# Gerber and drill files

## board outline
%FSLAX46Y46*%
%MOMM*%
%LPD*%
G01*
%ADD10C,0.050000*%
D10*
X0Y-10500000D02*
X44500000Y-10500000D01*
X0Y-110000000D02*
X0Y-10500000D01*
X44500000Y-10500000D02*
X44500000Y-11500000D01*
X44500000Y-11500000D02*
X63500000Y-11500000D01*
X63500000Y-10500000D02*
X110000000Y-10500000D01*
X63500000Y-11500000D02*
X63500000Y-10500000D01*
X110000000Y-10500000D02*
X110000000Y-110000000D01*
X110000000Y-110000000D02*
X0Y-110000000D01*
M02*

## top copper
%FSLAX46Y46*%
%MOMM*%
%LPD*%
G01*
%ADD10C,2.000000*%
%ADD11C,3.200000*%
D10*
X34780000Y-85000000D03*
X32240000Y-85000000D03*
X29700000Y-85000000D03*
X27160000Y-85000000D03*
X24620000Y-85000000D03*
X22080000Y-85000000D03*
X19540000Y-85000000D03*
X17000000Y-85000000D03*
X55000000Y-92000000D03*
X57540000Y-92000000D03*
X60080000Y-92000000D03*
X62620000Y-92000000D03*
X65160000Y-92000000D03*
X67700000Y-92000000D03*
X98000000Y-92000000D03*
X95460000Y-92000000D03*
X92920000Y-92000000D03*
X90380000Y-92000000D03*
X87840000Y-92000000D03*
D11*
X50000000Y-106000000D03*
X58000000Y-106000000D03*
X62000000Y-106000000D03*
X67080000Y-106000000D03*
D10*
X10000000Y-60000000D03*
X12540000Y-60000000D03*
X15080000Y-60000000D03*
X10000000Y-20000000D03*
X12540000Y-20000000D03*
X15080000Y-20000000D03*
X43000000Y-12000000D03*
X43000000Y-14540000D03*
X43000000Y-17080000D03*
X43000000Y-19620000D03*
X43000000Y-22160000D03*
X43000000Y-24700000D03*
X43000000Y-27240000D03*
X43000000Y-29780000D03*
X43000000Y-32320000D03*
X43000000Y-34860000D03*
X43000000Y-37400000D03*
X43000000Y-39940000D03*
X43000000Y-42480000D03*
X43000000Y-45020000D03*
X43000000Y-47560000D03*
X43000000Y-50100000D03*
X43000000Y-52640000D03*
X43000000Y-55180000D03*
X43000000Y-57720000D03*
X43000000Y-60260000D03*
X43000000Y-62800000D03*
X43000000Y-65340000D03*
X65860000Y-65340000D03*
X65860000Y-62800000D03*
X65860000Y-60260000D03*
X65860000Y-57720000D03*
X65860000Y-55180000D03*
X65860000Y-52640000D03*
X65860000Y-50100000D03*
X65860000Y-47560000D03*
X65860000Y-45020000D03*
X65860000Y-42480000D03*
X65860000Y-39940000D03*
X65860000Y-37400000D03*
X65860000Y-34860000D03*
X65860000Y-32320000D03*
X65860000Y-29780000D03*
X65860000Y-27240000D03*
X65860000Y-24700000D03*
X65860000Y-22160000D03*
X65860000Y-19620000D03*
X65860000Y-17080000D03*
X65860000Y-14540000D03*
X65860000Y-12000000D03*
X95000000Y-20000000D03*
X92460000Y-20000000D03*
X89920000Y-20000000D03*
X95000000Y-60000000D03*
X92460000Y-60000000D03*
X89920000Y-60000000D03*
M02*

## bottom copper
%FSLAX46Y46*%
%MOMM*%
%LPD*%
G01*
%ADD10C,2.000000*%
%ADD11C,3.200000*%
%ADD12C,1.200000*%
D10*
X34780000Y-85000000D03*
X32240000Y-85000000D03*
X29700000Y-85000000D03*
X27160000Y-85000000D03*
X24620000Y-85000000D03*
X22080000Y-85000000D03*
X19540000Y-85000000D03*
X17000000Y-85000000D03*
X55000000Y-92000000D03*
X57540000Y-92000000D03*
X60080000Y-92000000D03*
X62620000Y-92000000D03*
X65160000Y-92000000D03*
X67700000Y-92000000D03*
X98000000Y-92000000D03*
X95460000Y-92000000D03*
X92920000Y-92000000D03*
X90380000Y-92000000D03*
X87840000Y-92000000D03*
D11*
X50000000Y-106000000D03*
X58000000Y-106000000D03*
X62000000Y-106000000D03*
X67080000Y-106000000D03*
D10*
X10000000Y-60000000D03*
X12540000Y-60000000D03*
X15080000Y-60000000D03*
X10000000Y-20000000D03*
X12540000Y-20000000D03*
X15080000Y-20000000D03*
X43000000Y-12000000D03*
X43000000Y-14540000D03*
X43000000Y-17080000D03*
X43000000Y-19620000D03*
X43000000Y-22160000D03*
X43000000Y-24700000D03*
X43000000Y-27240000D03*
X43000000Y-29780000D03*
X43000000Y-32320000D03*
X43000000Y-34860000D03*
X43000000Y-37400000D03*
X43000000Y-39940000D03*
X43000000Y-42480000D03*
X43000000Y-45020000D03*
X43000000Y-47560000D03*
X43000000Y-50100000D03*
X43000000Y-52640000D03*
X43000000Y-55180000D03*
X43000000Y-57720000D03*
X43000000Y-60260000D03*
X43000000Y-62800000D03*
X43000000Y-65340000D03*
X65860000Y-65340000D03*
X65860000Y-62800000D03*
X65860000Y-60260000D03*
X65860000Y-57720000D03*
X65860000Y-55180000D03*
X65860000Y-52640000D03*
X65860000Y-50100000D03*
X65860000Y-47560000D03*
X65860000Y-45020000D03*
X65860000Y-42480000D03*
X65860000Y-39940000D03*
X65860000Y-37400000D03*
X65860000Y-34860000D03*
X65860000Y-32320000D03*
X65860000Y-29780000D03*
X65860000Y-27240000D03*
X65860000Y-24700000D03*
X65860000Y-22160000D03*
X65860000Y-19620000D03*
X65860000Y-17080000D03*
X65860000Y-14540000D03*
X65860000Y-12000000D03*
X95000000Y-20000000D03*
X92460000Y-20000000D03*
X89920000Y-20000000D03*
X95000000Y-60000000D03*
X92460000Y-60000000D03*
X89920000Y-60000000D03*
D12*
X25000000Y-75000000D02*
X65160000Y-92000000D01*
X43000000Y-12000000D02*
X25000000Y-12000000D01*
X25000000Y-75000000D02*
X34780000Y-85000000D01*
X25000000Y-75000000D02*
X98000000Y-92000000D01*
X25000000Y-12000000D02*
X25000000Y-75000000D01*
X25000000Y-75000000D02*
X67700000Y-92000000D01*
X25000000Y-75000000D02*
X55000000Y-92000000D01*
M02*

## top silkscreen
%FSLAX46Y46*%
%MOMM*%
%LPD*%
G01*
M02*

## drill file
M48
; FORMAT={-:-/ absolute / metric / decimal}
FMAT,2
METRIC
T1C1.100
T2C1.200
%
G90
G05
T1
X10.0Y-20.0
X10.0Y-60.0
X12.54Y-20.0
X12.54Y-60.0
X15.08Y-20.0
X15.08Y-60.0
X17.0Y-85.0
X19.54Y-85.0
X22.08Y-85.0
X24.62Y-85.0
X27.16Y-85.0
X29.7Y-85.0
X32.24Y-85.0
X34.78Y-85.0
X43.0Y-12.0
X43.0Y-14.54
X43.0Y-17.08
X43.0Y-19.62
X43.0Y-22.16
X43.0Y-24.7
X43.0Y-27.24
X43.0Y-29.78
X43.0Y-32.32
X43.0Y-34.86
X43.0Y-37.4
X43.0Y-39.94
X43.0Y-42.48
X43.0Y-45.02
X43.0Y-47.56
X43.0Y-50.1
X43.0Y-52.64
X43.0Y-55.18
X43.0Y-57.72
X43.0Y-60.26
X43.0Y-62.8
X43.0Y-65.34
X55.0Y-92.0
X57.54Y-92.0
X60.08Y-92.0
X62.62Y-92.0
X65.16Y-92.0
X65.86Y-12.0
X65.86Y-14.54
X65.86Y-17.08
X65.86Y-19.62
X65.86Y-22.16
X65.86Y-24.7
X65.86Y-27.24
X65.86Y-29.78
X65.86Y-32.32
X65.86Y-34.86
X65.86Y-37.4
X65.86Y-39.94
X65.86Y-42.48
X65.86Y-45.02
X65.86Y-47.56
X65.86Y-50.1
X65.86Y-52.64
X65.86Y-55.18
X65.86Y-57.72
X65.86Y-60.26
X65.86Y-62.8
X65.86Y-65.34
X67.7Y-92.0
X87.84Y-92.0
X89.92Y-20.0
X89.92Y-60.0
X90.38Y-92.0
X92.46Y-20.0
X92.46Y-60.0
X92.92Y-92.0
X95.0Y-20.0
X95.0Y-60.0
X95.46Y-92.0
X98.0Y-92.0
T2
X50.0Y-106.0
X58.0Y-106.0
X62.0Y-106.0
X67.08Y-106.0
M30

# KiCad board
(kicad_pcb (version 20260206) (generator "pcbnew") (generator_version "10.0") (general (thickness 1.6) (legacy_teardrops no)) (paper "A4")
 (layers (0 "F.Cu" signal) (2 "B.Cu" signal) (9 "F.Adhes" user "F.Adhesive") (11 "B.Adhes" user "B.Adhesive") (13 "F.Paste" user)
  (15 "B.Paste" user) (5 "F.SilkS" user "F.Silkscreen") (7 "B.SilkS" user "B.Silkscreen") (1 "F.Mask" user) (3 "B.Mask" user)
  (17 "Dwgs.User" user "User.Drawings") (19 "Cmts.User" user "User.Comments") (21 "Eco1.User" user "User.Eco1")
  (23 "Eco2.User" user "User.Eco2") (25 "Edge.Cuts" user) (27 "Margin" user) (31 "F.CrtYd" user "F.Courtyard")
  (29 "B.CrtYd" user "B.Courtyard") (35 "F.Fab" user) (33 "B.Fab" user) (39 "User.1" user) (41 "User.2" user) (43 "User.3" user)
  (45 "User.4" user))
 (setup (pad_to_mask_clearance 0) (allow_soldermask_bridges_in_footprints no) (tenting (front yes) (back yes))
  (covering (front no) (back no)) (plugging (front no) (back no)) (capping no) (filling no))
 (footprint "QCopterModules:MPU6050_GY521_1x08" (layer "F.Cu") (at 34.78 85 -90)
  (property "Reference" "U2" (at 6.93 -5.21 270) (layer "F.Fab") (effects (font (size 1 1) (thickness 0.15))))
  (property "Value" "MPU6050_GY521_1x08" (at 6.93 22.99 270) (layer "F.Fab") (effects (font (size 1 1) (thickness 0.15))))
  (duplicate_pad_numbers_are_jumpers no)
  (pad "1" thru_hole circle (at 0 0 270) (size 2 2) (drill 1.1) (layers "*.Cu" "*.Mask") (remove_unused_layers no) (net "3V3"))
  (pad "2" thru_hole circle (at 0 2.54 270) (size 2 2) (drill 1.1) (layers "*.Cu" "*.Mask") (remove_unused_layers no) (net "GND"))
  (pad "3" thru_hole circle (at 0 5.08 270) (size 2 2) (drill 1.1) (layers "*.Cu" "*.Mask") (remove_unused_layers no) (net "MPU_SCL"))
  (pad "4" thru_hole circle (at 0 7.62 270) (size 2 2) (drill 1.1) (layers "*.Cu" "*.Mask") (remove_unused_layers no) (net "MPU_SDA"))
  (pad "5" thru_hole circle (at 0 10.16 270) (size 2 2) (drill 1.1) (layers "*.Cu" "*.Mask") (remove_unused_layers no)
   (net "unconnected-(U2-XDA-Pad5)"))
  (pad "6" thru_hole circle (at 0 12.7 270) (size 2 2) (drill 1.1) (layers "*.Cu" "*.Mask") (remove_unused_layers no)
   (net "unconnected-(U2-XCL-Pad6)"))
  (pad "7" thru_hole circle (at 0 15.24 270) (size 2 2) (drill 1.1) (layers "*.Cu" "*.Mask") (remove_unused_layers no) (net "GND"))
  (pad "8" thru_hole circle (at 0 17.78 270) (size 2 2) (drill 1.1) (layers "*.Cu" "*.Mask") (remove_unused_layers no) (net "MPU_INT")))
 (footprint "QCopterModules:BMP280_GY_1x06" (layer "F.Cu") (at 55 92 90)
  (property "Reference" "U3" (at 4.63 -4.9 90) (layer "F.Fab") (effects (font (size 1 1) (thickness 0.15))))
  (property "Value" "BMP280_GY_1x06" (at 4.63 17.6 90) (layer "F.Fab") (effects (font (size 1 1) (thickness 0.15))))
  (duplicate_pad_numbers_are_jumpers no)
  (pad "1" thru_hole circle (at 0 0 90) (size 2 2) (drill 1.1) (layers "*.Cu" "*.Mask") (remove_unused_layers no) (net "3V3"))
  (pad "2" thru_hole circle (at 0 2.54 90) (size 2 2) (drill 1.1) (layers "*.Cu" "*.Mask") (remove_unused_layers no) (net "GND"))
  (pad "3" thru_hole circle (at 0 5.08 90) (size 2 2) (drill 1.1) (layers "*.Cu" "*.Mask") (remove_unused_layers no) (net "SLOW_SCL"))
  (pad "4" thru_hole circle (at 0 7.62 90) (size 2 2) (drill 1.1) (layers "*.Cu" "*.Mask") (remove_unused_layers no) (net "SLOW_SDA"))
  (pad "5" thru_hole circle (at 0 10.16 90) (size 2 2) (drill 1.1) (layers "*.Cu" "*.Mask") (remove_unused_layers no) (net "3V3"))
  (pad "6" thru_hole circle (at 0 12.7 90) (size 2 2) (drill 1.1) (layers "*.Cu" "*.Mask") (remove_unused_layers no) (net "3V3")))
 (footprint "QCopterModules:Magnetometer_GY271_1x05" (layer "F.Cu") (at 98 92 -90)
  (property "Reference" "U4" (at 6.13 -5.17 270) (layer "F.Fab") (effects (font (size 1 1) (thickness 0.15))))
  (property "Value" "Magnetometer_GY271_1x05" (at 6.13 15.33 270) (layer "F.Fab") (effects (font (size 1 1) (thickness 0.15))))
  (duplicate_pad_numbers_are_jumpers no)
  (pad "1" thru_hole circle (at 0 0 270) (size 2 2) (drill 1.1) (layers "*.Cu" "*.Mask") (remove_unused_layers no) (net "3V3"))
  (pad "2" thru_hole circle (at 0 2.54 270) (size 2 2) (drill 1.1) (layers "*.Cu" "*.Mask") (remove_unused_layers no) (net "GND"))
  (pad "3" thru_hole circle (at 0 5.08 270) (size 2 2) (drill 1.1) (layers "*.Cu" "*.Mask") (remove_unused_layers no) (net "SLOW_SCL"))
  (pad "4" thru_hole circle (at 0 7.62 270) (size 2 2) (drill 1.1) (layers "*.Cu" "*.Mask") (remove_unused_layers no) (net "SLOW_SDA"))
  (pad "5" thru_hole circle (at 0 10.16 270) (size 2 2) (drill 1.1) (layers "*.Cu" "*.Mask") (remove_unused_layers no) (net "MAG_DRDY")))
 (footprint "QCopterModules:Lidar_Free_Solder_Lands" (layer "F.Cu") (at 50 106)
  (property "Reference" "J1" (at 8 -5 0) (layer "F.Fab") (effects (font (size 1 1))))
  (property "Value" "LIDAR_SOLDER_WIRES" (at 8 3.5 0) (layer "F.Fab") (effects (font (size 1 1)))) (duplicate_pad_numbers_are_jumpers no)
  (pad "1" thru_hole circle (at 0 0) (size 3.2 3.2) (drill 1.2) (layers "*.Cu" "*.Mask") (remove_unused_layers no) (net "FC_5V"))
  (pad "2" thru_hole circle (at 8 0) (size 3.2 3.2) (drill 1.2) (layers "*.Cu" "*.Mask") (remove_unused_layers no) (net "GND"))
  (pad "3" thru_hole circle (at 12 0) (size 3.2 3.2) (drill 1.2) (layers "*.Cu" "*.Mask") (remove_unused_layers no) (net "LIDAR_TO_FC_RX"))
  (pad "4" thru_hole circle (at 17.08 0) (size 3.2 3.2) (drill 1.2) (layers "*.Cu" "*.Mask") (remove_unused_layers no)
   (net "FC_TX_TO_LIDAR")))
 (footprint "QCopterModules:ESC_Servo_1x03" (layer "F.Cu") (at 10 60 90)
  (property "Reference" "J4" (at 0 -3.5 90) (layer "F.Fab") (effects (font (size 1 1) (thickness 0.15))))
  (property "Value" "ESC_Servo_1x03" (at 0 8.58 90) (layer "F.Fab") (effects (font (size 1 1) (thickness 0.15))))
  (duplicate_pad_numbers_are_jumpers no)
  (pad "1" thru_hole circle (at 0 0 90) (size 2 2) (drill 1.1) (layers "*.Cu" "*.Mask") (remove_unused_layers no) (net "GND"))
  (pad "2" thru_hole circle (at 0 2.54 90) (size 2 2) (drill 1.1) (layers "*.Cu" "*.Mask") (remove_unused_layers no) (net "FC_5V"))
  (pad "3" thru_hole circle (at 0 5.08 90) (size 2 2) (drill 1.1) (layers "*.Cu" "*.Mask") (remove_unused_layers no) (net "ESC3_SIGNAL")))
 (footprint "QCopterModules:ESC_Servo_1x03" (layer "F.Cu") (at 10 20 90)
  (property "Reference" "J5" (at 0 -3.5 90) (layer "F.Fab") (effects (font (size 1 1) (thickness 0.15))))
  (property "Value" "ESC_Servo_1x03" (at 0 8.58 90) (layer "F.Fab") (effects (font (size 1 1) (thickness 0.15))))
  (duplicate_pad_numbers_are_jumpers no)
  (pad "1" thru_hole circle (at 0 0 90) (size 2 2) (drill 1.1) (layers "*.Cu" "*.Mask") (remove_unused_layers no) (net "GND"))
  (pad "2" thru_hole circle (at 0 2.54 90) (size 2 2) (drill 1.1) (layers "*.Cu" "*.Mask") (remove_unused_layers no)
   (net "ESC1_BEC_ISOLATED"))
  (pad "3" thru_hole circle (at 0 5.08 90) (size 2 2) (drill 1.1) (layers "*.Cu" "*.Mask") (remove_unused_layers no) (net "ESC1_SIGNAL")))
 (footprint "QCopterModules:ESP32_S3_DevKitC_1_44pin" (layer "F.Cu") (at 43 12)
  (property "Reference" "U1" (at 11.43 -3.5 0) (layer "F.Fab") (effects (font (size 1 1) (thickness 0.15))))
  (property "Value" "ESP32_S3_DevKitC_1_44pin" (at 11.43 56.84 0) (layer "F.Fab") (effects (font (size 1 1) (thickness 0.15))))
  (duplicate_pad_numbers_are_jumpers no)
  (pad "1" thru_hole circle (at 0 0) (size 2 2) (drill 1.1) (layers "*.Cu" "*.Mask") (remove_unused_layers no) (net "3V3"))
  (pad "2" thru_hole circle (at 0 2.54) (size 2 2) (drill 1.1) (layers "*.Cu" "*.Mask") (remove_unused_layers no))
  (pad "3" thru_hole circle (at 0 5.08) (size 2 2) (drill 1.1) (layers "*.Cu" "*.Mask") (remove_unused_layers no)
   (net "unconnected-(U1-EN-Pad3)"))
  (pad "4" thru_hole circle (at 0 7.62) (size 2 2) (drill 1.1) (layers "*.Cu" "*.Mask") (remove_unused_layers no) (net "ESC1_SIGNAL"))
  (pad "5" thru_hole circle (at 0 10.16) (size 2 2) (drill 1.1) (layers "*.Cu" "*.Mask") (remove_unused_layers no)
   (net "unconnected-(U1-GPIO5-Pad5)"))
  (pad "6" thru_hole circle (at 0 12.7) (size 2 2) (drill 1.1) (layers "*.Cu" "*.Mask") (remove_unused_layers no)
   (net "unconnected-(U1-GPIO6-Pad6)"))
  (pad "7" thru_hole circle (at 0 15.24) (size 2 2) (drill 1.1) (layers "*.Cu" "*.Mask") (remove_unused_layers no)
   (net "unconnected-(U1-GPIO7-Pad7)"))
  (pad "8" thru_hole circle (at 0 17.78) (size 2 2) (drill 1.1) (layers "*.Cu" "*.Mask") (remove_unused_layers no) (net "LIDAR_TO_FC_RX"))
  (pad "9" thru_hole circle (at 0 20.32) (size 2 2) (drill 1.1) (layers "*.Cu" "*.Mask") (remove_unused_layers no) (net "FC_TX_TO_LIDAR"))
  (pad "10" thru_hole circle (at 0 22.86) (size 2 2) (drill 1.1) (layers "*.Cu" "*.Mask") (remove_unused_layers no)
   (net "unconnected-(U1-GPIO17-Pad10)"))
  (pad "11" thru_hole circle (at 0 25.4) (size 2 2) (drill 1.1) (layers "*.Cu" "*.Mask") (remove_unused_layers no) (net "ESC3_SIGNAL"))
  (pad "12" thru_hole circle (at 0 27.94) (size 2 2) (drill 1.1) (layers "*.Cu" "*.Mask") (remove_unused_layers no)
   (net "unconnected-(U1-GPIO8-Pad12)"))
  (pad "13" thru_hole circle (at 0 30.48) (size 2 2) (drill 1.1) (layers "*.Cu" "*.Mask") (remove_unused_layers no)
   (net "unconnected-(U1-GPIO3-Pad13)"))
  (pad "14" thru_hole circle (at 0 33.02) (size 2 2) (drill 1.1) (layers "*.Cu" "*.Mask") (remove_unused_layers no)
   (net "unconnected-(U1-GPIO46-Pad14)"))
  (pad "15" thru_hole circle (at 0 35.56) (size 2 2) (drill 1.1) (layers "*.Cu" "*.Mask") (remove_unused_layers no)
   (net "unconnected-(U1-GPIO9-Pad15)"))
  (pad "16" thru_hole circle (at 0 38.1) (size 2 2) (drill 1.1) (layers "*.Cu" "*.Mask") (remove_unused_layers no)
   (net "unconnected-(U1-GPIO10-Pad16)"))
  (pad "17" thru_hole circle (at 0 40.64) (size 2 2) (drill 1.1) (layers "*.Cu" "*.Mask") (remove_unused_layers no)
   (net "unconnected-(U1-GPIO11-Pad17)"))
  (pad "18" thru_hole circle (at 0 43.18) (size 2 2) (drill 1.1) (layers "*.Cu" "*.Mask") (remove_unused_layers no) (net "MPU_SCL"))
  (pad "19" thru_hole circle (at 0 45.72) (size 2 2) (drill 1.1) (layers "*.Cu" "*.Mask") (remove_unused_layers no) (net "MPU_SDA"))
  (pad "20" thru_hole circle (at 0 48.26) (size 2 2) (drill 1.1) (layers "*.Cu" "*.Mask") (remove_unused_layers no) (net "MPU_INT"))
  (pad "21" thru_hole circle (at 0 50.8) (size 2 2) (drill 1.1) (layers "*.Cu" "*.Mask") (remove_unused_layers no) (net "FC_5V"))
  (pad "22" thru_hole circle (at 0 53.34) (size 2 2) (drill 1.1) (layers "*.Cu" "*.Mask") (remove_unused_layers no) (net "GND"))
  (pad "23" thru_hole circle (at 22.86 53.34) (size 2 2) (drill 1.1) (layers "*.Cu" "*.Mask") (remove_unused_layers no) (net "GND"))
  (pad "24" thru_hole circle (at 22.86 50.8) (size 2 2) (drill 1.1) (layers "*.Cu" "*.Mask") (remove_unused_layers no) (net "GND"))
  (pad "25" thru_hole circle (at 22.86 48.26) (size 2 2) (drill 1.1) (layers "*.Cu" "*.Mask") (remove_unused_layers no)
   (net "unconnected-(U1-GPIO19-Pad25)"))
  (pad "26" thru_hole circle (at 22.86 45.72) (size 2 2) (drill 1.1) (layers "*.Cu" "*.Mask") (remove_unused_layers no)
   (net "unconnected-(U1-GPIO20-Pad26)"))
  (pad "27" thru_hole circle (at 22.86 43.18) (size 2 2) (drill 1.1) (layers "*.Cu" "*.Mask") (remove_unused_layers no) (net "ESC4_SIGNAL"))
  (pad "28" thru_hole circle (at 22.86 40.64) (size 2 2) (drill 1.1) (layers "*.Cu" "*.Mask") (remove_unused_layers no)
   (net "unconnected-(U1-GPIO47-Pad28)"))
  (pad "29" thru_hole circle (at 22.86 38.1) (size 2 2) (drill 1.1) (layers "*.Cu" "*.Mask") (remove_unused_layers no)
   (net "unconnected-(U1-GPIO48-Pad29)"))
  (pad "30" thru_hole circle (at 22.86 35.56) (size 2 2) (drill 1.1) (layers "*.Cu" "*.Mask") (remove_unused_layers no)
   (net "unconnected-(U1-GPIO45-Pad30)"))
  (pad "31" thru_hole circle (at 22.86 33.02) (size 2 2) (drill 1.1) (layers "*.Cu" "*.Mask") (remove_unused_layers no)
   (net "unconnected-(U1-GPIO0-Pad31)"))
  (pad "32" thru_hole circle (at 22.86 30.48) (size 2 2) (drill 1.1) (layers "*.Cu" "*.Mask") (remove_unused_layers no)
   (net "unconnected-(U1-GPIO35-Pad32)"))
  (pad "33" thru_hole circle (at 22.86 27.94) (size 2 2) (drill 1.1) (layers "*.Cu" "*.Mask") (remove_unused_layers no)
   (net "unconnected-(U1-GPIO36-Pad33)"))
  (pad "34" thru_hole circle (at 22.86 25.4) (size 2 2) (drill 1.1) (layers "*.Cu" "*.Mask") (remove_unused_layers no)
   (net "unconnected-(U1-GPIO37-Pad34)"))
  (pad "35" thru_hole circle (at 22.86 22.86) (size 2 2) (drill 1.1) (layers "*.Cu" "*.Mask") (remove_unused_layers no)
   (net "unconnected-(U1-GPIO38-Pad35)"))
  (pad "36" thru_hole circle (at 22.86 20.32) (size 2 2) (drill 1.1) (layers "*.Cu" "*.Mask") (remove_unused_layers no) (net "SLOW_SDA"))
  (pad "37" thru_hole circle (at 22.86 17.78) (size 2 2) (drill 1.1) (layers "*.Cu" "*.Mask") (remove_unused_layers no) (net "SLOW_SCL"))
  (pad "38" thru_hole circle (at 22.86 15.24) (size 2 2) (drill 1.1) (layers "*.Cu" "*.Mask") (remove_unused_layers no) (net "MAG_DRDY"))
  (pad "39" thru_hole circle (at 22.86 12.7) (size 2 2) (drill 1.1) (layers "*.Cu" "*.Mask") (remove_unused_layers no)
   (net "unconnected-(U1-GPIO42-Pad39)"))
  (pad "40" thru_hole circle (at 22.86 10.16) (size 2 2) (drill 1.1) (layers "*.Cu" "*.Mask") (remove_unused_layers no) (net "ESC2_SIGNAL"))
  (pad "41" thru_hole circle (at 22.86 7.62) (size 2 2) (drill 1.1) (layers "*.Cu" "*.Mask") (remove_unused_layers no)
   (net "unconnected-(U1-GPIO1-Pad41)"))
  (pad "42" thru_hole circle (at 22.86 5.08) (size 2 2) (drill 1.1) (layers "*.Cu" "*.Mask") (remove_unused_layers no)
   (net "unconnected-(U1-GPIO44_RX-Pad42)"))
  (pad "43" thru_hole circle (at 22.86 2.54) (size 2 2) (drill 1.1) (layers "*.Cu" "*.Mask") (remove_unused_layers no)
   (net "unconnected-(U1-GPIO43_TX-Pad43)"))
  (pad "44" thru_hole circle (at 22.86 0) (size 2 2) (drill 1.1) (layers "*.Cu" "*.Mask") (remove_unused_layers no) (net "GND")))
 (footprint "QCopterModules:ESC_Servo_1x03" (layer "F.Cu") (at 95 20 -90)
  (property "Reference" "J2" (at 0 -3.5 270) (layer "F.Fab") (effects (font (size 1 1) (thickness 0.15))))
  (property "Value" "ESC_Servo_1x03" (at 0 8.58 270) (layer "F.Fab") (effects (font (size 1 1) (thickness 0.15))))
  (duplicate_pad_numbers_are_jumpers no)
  (pad "1" thru_hole circle (at 0 0 270) (size 2 2) (drill 1.1) (layers "*.Cu" "*.Mask") (remove_unused_layers no) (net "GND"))
  (pad "2" thru_hole circle (at 0 2.54 270) (size 2 2) (drill 1.1) (layers "*.Cu" "*.Mask") (remove_unused_layers no)
   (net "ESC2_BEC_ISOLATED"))
  (pad "3" thru_hole circle (at 0 5.08 270) (size 2 2) (drill 1.1) (layers "*.Cu" "*.Mask") (remove_unused_layers no) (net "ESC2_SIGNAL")))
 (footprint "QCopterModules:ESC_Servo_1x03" (layer "F.Cu") (at 95 60 -90)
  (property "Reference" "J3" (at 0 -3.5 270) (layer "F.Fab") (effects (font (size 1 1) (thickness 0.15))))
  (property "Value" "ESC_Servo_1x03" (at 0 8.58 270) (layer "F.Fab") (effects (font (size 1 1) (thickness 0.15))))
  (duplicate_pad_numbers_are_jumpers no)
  (pad "1" thru_hole circle (at 0 0 270) (size 2 2) (drill 1.1) (layers "*.Cu" "*.Mask") (remove_unused_layers no) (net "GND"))
  (pad "2" thru_hole circle (at 0 2.54 270) (size 2 2) (drill 1.1) (layers "*.Cu" "*.Mask") (remove_unused_layers no)
   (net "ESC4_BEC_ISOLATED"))
  (pad "3" thru_hole circle (at 0 5.08 270) (size 2 2) (drill 1.1) (layers "*.Cu" "*.Mask") (remove_unused_layers no) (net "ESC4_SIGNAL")))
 (gr_line (start 0 10.5) (end 44.5 10.5) (stroke (width 0.05) (type default)) (layer "Edge.Cuts"))
 (gr_line (start 0 110) (end 0 10.5) (stroke (width 0.05) (type default)) (layer "Edge.Cuts"))
 (gr_line (start 44.5 10.5) (end 44.5 11.5) (stroke (width 0.05) (type default)) (layer "Edge.Cuts"))
 (gr_line (start 44.5 11.5) (end 63.5 11.5) (stroke (width 0.05) (type default)) (layer "Edge.Cuts"))
 (gr_line (start 63.5 10.5) (end 110 10.5) (stroke (width 0.05) (type default)) (layer "Edge.Cuts"))
 (gr_line (start 63.5 11.5) (end 63.5 10.5) (stroke (width 0.05) (type default)) (layer "Edge.Cuts"))
 (gr_line (start 110 10.5) (end 110 110) (stroke (width 0.05) (type default)) (layer "Edge.Cuts"))
 (gr_line (start 110 110) (end 0 110) (stroke (width 0.05) (type default)) (layer "Edge.Cuts"))
 (segment (start 25 75) (end 65.16 92) (width 1.2) (layer "B.Cu") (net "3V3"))
 (segment (start 43 12) (end 25 12) (width 1.2) (layer "B.Cu") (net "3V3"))
 (segment (start 25 75) (end 34.78 85) (width 1.2) (layer "B.Cu") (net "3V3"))
 (segment (start 25 75) (end 98 92) (width 1.2) (layer "B.Cu") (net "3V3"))
 (segment (start 25 12) (end 25 75) (width 1.2) (layer "B.Cu") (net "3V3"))
 (segment (start 25 75) (end 67.7 92) (width 1.2) (layer "B.Cu") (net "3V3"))
 (segment (start 25 75) (end 55 92) (width 1.2) (layer "B.Cu") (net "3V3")))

